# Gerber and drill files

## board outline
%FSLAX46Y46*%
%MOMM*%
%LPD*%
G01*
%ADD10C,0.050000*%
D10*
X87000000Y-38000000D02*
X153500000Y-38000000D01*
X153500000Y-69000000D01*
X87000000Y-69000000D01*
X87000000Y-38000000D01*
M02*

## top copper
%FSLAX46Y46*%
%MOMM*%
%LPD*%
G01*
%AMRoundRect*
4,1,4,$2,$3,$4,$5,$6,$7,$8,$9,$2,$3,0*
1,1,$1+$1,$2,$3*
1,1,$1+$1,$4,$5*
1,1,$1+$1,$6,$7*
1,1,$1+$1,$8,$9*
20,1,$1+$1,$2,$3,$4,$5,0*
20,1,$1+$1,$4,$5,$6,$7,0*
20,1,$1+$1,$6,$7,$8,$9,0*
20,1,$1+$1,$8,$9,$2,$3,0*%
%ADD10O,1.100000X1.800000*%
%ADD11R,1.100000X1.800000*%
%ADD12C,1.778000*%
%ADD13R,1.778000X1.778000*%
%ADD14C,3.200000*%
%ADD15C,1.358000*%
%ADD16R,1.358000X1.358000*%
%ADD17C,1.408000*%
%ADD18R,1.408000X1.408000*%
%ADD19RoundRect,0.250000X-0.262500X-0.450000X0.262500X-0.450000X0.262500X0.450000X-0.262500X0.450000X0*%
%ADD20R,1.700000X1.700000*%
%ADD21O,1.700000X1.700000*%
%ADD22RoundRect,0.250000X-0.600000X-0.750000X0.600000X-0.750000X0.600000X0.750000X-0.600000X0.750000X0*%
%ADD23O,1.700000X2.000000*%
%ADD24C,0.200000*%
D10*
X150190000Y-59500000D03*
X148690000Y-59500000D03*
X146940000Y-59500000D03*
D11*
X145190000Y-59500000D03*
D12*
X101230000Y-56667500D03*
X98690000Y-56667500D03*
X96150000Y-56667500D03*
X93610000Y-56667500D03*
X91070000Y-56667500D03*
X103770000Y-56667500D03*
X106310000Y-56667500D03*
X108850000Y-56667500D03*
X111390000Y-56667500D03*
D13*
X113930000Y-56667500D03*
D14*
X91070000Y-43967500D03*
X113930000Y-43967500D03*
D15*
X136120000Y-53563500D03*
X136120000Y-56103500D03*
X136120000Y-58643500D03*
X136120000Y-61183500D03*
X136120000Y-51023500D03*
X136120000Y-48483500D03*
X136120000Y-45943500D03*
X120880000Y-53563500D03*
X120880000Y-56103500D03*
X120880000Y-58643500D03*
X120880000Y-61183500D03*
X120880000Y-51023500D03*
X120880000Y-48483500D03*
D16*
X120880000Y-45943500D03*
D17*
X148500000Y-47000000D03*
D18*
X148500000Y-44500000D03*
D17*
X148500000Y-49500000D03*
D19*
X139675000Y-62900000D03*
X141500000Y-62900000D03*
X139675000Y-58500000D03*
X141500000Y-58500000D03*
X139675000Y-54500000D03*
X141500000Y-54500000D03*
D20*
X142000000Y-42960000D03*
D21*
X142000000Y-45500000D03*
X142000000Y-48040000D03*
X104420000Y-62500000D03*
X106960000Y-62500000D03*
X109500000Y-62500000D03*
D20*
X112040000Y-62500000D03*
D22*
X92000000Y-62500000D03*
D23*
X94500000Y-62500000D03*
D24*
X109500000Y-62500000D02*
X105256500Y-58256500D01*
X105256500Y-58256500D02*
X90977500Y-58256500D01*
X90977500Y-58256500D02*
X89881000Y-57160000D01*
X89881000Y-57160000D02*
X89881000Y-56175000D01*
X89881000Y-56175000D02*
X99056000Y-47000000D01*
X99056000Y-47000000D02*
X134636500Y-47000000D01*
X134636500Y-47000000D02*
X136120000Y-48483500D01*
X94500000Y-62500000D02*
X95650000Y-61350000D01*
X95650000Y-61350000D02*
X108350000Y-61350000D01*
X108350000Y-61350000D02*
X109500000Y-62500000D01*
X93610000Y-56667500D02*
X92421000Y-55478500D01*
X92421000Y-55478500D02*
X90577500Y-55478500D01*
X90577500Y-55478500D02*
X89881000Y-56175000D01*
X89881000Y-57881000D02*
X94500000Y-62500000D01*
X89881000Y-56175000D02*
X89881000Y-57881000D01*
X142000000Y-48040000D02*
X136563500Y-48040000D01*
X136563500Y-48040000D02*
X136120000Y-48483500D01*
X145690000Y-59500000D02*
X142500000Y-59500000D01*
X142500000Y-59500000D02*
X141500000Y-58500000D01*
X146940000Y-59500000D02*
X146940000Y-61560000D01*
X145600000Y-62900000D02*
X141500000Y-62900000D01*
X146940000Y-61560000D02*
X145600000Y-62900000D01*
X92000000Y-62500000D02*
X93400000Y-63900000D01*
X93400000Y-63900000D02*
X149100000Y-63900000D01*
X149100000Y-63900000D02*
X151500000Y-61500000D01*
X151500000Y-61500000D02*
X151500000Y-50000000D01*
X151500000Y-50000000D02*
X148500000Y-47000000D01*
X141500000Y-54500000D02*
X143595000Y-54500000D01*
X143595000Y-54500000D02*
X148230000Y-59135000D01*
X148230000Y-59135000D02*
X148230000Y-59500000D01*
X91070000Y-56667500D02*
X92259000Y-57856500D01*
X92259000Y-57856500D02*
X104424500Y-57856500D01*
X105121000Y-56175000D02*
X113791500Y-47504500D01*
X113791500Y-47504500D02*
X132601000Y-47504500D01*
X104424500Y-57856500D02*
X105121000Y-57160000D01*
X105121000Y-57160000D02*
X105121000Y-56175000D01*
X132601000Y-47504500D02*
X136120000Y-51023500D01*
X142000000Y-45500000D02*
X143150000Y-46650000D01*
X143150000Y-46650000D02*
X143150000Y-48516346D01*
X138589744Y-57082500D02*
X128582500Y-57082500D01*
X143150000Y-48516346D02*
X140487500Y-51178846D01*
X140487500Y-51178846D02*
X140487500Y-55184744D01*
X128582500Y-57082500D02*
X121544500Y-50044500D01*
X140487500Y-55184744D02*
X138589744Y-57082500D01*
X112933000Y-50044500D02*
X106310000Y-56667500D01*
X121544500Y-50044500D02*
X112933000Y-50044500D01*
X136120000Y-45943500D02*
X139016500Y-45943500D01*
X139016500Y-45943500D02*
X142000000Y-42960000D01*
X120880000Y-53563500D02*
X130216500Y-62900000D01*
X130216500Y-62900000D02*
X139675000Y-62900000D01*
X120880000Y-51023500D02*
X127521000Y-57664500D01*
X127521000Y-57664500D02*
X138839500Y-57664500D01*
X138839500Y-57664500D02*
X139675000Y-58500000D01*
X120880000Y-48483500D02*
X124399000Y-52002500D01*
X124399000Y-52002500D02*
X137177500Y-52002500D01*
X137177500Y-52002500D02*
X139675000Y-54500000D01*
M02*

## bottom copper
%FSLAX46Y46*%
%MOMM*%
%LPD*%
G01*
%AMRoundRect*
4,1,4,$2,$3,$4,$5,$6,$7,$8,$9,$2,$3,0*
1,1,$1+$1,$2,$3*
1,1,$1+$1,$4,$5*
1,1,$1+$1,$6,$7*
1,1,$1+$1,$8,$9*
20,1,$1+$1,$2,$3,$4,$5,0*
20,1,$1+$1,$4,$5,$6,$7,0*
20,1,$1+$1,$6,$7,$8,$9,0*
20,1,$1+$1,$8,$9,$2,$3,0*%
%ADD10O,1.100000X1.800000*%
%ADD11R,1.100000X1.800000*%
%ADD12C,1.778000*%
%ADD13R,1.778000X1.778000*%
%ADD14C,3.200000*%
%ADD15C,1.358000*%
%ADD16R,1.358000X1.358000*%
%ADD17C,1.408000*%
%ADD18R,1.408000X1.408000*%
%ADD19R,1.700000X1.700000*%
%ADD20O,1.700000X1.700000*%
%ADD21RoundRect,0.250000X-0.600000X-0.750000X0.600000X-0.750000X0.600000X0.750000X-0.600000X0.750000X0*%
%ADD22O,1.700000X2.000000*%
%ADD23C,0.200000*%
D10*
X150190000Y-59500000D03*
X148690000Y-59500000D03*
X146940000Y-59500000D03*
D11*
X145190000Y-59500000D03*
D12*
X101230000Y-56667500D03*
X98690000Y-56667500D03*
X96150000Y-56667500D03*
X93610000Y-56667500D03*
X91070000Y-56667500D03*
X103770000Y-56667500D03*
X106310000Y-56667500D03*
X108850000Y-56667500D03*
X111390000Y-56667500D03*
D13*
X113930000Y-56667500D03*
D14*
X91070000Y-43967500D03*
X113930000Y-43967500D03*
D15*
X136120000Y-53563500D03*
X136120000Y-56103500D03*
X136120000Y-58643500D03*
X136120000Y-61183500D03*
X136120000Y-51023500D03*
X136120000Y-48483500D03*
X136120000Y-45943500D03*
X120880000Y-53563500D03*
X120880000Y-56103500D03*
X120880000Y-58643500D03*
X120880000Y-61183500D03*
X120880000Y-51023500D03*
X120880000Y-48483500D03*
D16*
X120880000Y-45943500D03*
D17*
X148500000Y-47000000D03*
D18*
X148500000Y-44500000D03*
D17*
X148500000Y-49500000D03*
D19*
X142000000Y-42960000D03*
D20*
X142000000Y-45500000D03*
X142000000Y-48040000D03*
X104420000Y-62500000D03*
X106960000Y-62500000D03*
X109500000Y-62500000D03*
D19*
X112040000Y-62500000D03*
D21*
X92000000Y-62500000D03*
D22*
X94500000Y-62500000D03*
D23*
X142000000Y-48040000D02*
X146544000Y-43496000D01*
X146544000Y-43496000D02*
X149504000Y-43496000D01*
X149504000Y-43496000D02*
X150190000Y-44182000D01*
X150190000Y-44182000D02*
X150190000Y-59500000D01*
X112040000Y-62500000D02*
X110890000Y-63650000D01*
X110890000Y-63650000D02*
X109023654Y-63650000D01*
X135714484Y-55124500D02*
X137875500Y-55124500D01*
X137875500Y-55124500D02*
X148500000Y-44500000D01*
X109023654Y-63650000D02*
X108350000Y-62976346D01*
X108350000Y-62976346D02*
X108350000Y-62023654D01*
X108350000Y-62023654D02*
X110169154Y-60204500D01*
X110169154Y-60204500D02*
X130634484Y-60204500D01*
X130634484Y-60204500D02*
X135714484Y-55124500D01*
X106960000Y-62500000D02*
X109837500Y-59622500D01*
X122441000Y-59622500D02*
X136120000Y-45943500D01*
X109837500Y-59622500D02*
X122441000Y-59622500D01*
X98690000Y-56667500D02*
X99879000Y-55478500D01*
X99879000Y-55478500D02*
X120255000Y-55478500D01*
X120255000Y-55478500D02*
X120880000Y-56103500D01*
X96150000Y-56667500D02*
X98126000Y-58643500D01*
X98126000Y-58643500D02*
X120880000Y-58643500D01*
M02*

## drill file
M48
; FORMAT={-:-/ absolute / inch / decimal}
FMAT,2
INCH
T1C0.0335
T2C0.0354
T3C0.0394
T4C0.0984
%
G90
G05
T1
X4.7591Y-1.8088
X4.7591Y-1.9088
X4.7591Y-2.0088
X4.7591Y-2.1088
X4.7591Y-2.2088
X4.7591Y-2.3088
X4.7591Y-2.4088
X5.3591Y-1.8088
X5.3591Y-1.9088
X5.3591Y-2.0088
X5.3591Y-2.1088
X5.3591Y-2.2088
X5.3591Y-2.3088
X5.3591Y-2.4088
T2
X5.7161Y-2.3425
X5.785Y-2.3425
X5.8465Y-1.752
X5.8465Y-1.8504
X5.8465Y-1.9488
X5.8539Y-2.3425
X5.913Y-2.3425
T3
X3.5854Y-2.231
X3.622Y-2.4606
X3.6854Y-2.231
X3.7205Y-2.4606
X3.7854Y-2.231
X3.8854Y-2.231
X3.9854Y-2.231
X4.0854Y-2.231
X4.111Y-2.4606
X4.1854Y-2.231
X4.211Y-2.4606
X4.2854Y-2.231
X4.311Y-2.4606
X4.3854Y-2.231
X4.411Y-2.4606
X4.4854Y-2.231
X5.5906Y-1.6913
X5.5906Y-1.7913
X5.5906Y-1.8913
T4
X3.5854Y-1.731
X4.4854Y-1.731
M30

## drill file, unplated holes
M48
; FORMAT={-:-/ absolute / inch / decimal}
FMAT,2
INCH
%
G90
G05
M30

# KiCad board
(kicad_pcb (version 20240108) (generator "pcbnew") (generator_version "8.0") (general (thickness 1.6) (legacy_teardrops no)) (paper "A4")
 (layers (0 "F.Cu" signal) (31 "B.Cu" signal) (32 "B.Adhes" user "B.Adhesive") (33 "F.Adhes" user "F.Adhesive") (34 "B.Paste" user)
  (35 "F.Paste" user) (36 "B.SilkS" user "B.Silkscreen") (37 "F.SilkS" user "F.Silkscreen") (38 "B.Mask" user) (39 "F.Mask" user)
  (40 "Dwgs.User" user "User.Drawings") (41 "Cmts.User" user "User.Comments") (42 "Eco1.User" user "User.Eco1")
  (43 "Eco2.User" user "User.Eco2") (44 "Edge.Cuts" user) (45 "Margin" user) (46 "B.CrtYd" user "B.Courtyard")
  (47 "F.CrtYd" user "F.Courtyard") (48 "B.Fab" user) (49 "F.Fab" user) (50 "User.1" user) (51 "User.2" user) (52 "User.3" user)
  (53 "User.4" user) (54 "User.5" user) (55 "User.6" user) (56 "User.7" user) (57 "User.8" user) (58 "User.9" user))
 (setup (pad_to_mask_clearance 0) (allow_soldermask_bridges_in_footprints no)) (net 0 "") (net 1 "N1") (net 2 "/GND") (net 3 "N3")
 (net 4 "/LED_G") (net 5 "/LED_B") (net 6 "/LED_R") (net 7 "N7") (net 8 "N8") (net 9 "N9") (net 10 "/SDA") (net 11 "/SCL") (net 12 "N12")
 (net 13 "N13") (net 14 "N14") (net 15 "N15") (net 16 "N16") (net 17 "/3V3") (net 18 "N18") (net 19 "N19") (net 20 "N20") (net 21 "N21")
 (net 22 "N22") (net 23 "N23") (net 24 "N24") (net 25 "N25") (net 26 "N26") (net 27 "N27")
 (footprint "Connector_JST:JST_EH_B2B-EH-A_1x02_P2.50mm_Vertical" (layer "F.Cu") (at 92 62.5)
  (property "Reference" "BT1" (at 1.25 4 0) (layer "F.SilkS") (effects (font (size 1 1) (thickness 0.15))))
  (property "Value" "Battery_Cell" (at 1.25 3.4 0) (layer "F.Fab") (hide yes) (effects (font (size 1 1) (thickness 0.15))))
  (pad "1" thru_hole roundrect (at 0 0) (size 1.7 2) (drill 1) (layers "*.Cu" "*.Mask") (remove_unused_layers no)
   (roundrect_rratio 0.147059) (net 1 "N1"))
  (pad "2" thru_hole oval (at 2.5 0) (size 1.7 2) (drill 1) (layers "*.Cu" "*.Mask") (remove_unused_layers no) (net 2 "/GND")))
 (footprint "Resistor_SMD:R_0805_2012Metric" (layer "F.Cu") (at 140.5875 58.5)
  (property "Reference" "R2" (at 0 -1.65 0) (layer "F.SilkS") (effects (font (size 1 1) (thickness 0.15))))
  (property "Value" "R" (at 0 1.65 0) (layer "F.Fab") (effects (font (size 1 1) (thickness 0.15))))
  (pad "1" smd roundrect (at -0.9125 0) (size 1.025 1.4) (layers "F.Cu" "F.Paste" "F.Mask") (roundrect_rratio 0.243902) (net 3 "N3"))
  (pad "2" smd roundrect (at 0.9125 0) (size 1.025 1.4) (layers "F.Cu" "F.Paste" "F.Mask") (roundrect_rratio 0.243902) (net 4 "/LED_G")))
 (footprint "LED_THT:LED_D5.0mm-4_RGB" (layer "F.Cu") (at 145.69 59.5)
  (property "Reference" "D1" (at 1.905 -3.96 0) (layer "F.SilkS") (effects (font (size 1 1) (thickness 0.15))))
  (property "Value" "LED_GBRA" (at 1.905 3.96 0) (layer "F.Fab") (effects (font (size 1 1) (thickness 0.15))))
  (pad "1" thru_hole rect (at -0.5 0) (size 1.1 1.8) (drill 0.9) (layers "*.Cu" "*.Mask") (remove_unused_layers no) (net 4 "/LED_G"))
  (pad "2" thru_hole oval (at 1.25 0) (size 1.1 1.8) (drill 0.9) (layers "*.Cu" "*.Mask") (remove_unused_layers no) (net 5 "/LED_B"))
  (pad "3" thru_hole oval (at 3 0) (size 1.1 1.8) (drill 0.9) (layers "*.Cu" "*.Mask") (remove_unused_layers no) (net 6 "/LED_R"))
  (pad "4" thru_hole oval (at 4.5 0) (size 1.1 1.8) (drill 0.9) (layers "*.Cu" "*.Mask") (remove_unused_layers no) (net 2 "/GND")))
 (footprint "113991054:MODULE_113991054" (layer "F.Cu") (at 128.5 53.5)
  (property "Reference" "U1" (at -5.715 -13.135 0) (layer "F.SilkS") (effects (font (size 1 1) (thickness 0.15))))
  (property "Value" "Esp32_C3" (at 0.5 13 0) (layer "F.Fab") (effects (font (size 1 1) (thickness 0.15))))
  (pad "1" thru_hole rect (at -7.62 -7.5565) (size 1.358 1.358) (drill 0.85) (layers "*.Cu" "*.Mask") (remove_unused_layers no) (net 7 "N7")
   (solder_mask_margin 0.102))
  (pad "2" thru_hole circle (at -7.62 -5.0165) (size 1.358 1.358) (drill 0.85) (layers "*.Cu" "*.Mask") (remove_unused_layers no)
   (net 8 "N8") (solder_mask_margin 0.102))
  (pad "3" thru_hole circle (at -7.62 -2.4765) (size 1.358 1.358) (drill 0.85) (layers "*.Cu" "*.Mask") (remove_unused_layers no)
   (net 3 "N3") (solder_mask_margin 0.102))
  (pad "4" thru_hole circle (at -7.62 0.0635) (size 1.358 1.358) (drill 0.85) (layers "*.Cu" "*.Mask") (remove_unused_layers no)
   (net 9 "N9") (solder_mask_margin 0.102))
  (pad "5" thru_hole circle (at -7.62 2.6035) (size 1.358 1.358) (drill 0.85) (layers "*.Cu" "*.Mask") (remove_unused_layers no)
   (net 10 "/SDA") (solder_mask_margin 0.102))
  (pad "6" thru_hole circle (at -7.62 5.1435) (size 1.358 1.358) (drill 0.85) (layers "*.Cu" "*.Mask") (remove_unused_layers no)
   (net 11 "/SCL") (solder_mask_margin 0.102))
  (pad "7" thru_hole circle (at -7.62 7.6835) (size 1.358 1.358) (drill 0.85) (layers "*.Cu" "*.Mask") (remove_unused_layers no)
   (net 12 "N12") (solder_mask_margin 0.102))
  (pad "8" thru_hole circle (at 7.62 7.6835) (size 1.358 1.358) (drill 0.85) (layers "*.Cu" "*.Mask") (remove_unused_layers no)
   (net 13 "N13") (solder_mask_margin 0.102))
  (pad "9" thru_hole circle (at 7.62 5.1435) (size 1.358 1.358) (drill 0.85) (layers "*.Cu" "*.Mask") (remove_unused_layers no)
   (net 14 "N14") (solder_mask_margin 0.102))
  (pad "10" thru_hole circle (at 7.62 2.6035) (size 1.358 1.358) (drill 0.85) (layers "*.Cu" "*.Mask") (remove_unused_layers no)
   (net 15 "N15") (solder_mask_margin 0.102))
  (pad "11" thru_hole circle (at 7.62 0.0635) (size 1.358 1.358) (drill 0.85) (layers "*.Cu" "*.Mask") (remove_unused_layers no)
   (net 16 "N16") (solder_mask_margin 0.102))
  (pad "12" thru_hole circle (at 7.62 -2.4765) (size 1.358 1.358) (drill 0.85) (layers "*.Cu" "*.Mask") (remove_unused_layers no)
   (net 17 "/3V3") (solder_mask_margin 0.102))
  (pad "13" thru_hole circle (at 7.62 -5.0165) (size 1.358 1.358) (drill 0.85) (layers "*.Cu" "*.Mask") (remove_unused_layers no)
   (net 2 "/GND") (solder_mask_margin 0.102))
  (pad "14" thru_hole circle (at 7.62 -7.5565) (size 1.358 1.358) (drill 0.85) (layers "*.Cu" "*.Mask") (remove_unused_layers no)
   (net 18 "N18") (solder_mask_margin 0.102)))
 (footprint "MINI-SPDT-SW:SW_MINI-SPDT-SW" (layer "F.Cu") (at 148.5 47 -90)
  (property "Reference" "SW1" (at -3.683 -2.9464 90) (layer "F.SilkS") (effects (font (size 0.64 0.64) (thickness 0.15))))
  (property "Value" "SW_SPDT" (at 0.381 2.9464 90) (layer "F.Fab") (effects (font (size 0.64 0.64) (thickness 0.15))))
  (pad "1" thru_hole rect (at -2.5 0 270) (size 1.408 1.408) (drill 0.9) (layers "*.Cu" "*.Mask") (remove_unused_layers no) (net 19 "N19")
   (solder_mask_margin 0.102))
  (pad "2" thru_hole circle (at 0 0 270) (size 1.408 1.408) (drill 0.9) (layers "*.Cu" "*.Mask") (remove_unused_layers no) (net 1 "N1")
   (solder_mask_margin 0.102))
  (pad "3" thru_hole circle (at 2.5 0 270) (size 1.408 1.408) (drill 0.9) (layers "*.Cu" "*.Mask") (remove_unused_layers no) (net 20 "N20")
   (solder_mask_margin 0.102)))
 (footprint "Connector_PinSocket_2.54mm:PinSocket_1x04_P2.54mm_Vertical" (layer "F.Cu") (at 112.04 62.5 -90)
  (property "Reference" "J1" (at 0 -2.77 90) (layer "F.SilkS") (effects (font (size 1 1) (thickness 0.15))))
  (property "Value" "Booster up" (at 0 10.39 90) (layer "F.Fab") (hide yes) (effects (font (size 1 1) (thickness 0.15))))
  (pad "1" thru_hole rect (at 0 0 270) (size 1.7 1.7) (drill 1) (layers "*.Cu" "*.Mask") (remove_unused_layers no) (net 19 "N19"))
  (pad "2" thru_hole oval (at 0 2.54 270) (size 1.7 1.7) (drill 1) (layers "*.Cu" "*.Mask") (remove_unused_layers no) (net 2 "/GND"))
  (pad "3" thru_hole oval (at 0 5.08 270) (size 1.7 1.7) (drill 1) (layers "*.Cu" "*.Mask") (remove_unused_layers no) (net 18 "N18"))
  (pad "4" thru_hole oval (at 0 7.62 270) (size 1.7 1.7) (drill 1) (layers "*.Cu" "*.Mask") (remove_unused_layers no) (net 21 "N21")))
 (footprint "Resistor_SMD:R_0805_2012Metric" (layer "F.Cu") (at 140.5875 54.5)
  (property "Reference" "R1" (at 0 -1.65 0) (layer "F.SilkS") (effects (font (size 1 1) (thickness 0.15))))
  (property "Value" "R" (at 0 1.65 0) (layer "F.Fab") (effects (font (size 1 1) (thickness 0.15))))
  (pad "1" smd roundrect (at -0.9125 0) (size 1.025 1.4) (layers "F.Cu" "F.Paste" "F.Mask") (roundrect_rratio 0.243902) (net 8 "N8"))
  (pad "2" smd roundrect (at 0.9125 0) (size 1.025 1.4) (layers "F.Cu" "F.Paste" "F.Mask") (roundrect_rratio 0.243902) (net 6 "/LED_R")))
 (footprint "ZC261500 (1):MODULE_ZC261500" (layer "F.Cu") (at 102.5 50)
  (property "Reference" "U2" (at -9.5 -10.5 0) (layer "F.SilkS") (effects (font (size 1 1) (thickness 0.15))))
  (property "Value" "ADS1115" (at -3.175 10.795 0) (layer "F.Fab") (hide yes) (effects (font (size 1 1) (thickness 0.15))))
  (pad "1" thru_hole rect (at 11.43 6.6675) (size 1.778 1.778) (drill 1) (layers "*.Cu" "*.Mask") (remove_unused_layers no) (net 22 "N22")
   (solder_mask_margin 0.102))
  (pad "2" thru_hole circle (at 8.89 6.6675) (size 1.778 1.778) (drill 1) (layers "*.Cu" "*.Mask") (remove_unused_layers no) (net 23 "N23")
   (solder_mask_margin 0.102))
  (pad "3" thru_hole circle (at 6.35 6.6675) (size 1.778 1.778) (drill 1) (layers "*.Cu" "*.Mask") (remove_unused_layers no) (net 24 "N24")
   (solder_mask_margin 0.102))
  (pad "4" thru_hole circle (at 3.81 6.6675) (size 1.778 1.778) (drill 1) (layers "*.Cu" "*.Mask") (remove_unused_layers no) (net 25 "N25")
   (solder_mask_margin 0.102))
  (pad "5" thru_hole circle (at 1.27 6.6675) (size 1.778 1.778) (drill 1) (layers "*.Cu" "*.Mask") (remove_unused_layers no) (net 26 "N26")
   (solder_mask_margin 0.102))
  (pad "6" thru_hole circle (at -1.27 6.6675) (size 1.778 1.778) (drill 1) (layers "*.Cu" "*.Mask") (remove_unused_layers no) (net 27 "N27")
   (solder_mask_margin 0.102))
  (pad "7" thru_hole circle (at -3.81 6.6675) (size 1.778 1.778) (drill 1) (layers "*.Cu" "*.Mask") (remove_unused_layers no)
   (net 10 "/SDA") (solder_mask_margin 0.102))
  (pad "8" thru_hole circle (at -6.35 6.6675) (size 1.778 1.778) (drill 1) (layers "*.Cu" "*.Mask") (remove_unused_layers no)
   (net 11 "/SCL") (solder_mask_margin 0.102))
  (pad "9" thru_hole circle (at -8.89 6.6675) (size 1.778 1.778) (drill 1) (layers "*.Cu" "*.Mask") (remove_unused_layers no) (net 2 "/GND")
   (solder_mask_margin 0.102))
  (pad "10" thru_hole circle (at -11.43 6.6675) (size 1.778 1.778) (drill 1) (layers "*.Cu" "*.Mask") (remove_unused_layers no)
   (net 17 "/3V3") (solder_mask_margin 0.102))
  (pad "P1" thru_hole circle (at -11.43 -6.0325) (size 3.2 3.2) (drill 2.5) (layers "*.Cu" "*.Mask") (remove_unused_layers no)
   (solder_mask_margin 0.102))
  (pad "P2" thru_hole circle (at 11.43 -6.0325) (size 3.2 3.2) (drill 2.5) (layers "*.Cu" "*.Mask") (remove_unused_layers no)
   (solder_mask_margin 0.102)))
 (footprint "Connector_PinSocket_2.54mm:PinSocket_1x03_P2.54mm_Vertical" (layer "F.Cu") (at 142 42.96)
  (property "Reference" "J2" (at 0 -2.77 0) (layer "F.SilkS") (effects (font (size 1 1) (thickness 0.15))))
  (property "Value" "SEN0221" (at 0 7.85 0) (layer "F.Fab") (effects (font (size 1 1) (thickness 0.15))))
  (pad "1" thru_hole rect (at 0 0) (size 1.7 1.7) (drill 1) (layers "*.Cu" "*.Mask") (remove_unused_layers no) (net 18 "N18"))
  (pad "2" thru_hole oval (at 0 2.54) (size 1.7 1.7) (drill 1) (layers "*.Cu" "*.Mask") (remove_unused_layers no) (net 25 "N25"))
  (pad "3" thru_hole oval (at 0 5.08) (size 1.7 1.7) (drill 1) (layers "*.Cu" "*.Mask") (remove_unused_layers no) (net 2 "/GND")))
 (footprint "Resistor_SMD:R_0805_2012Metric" (layer "F.Cu") (at 140.5875 62.9)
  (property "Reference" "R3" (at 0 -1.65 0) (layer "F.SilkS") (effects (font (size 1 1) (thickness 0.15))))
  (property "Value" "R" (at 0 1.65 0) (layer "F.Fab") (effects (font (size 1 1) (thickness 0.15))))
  (pad "1" smd roundrect (at -0.9125 0) (size 1.025 1.4) (layers "F.Cu" "F.Paste" "F.Mask") (roundrect_rratio 0.243902) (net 9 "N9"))
  (pad "2" smd roundrect (at 0.9125 0) (size 1.025 1.4) (layers "F.Cu" "F.Paste" "F.Mask") (roundrect_rratio 0.243902) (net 5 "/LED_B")))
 (gr_rect (start 87 38) (end 153.5 69) (stroke (width 0.05) (type default)) (fill none) (layer "Edge.Cuts"))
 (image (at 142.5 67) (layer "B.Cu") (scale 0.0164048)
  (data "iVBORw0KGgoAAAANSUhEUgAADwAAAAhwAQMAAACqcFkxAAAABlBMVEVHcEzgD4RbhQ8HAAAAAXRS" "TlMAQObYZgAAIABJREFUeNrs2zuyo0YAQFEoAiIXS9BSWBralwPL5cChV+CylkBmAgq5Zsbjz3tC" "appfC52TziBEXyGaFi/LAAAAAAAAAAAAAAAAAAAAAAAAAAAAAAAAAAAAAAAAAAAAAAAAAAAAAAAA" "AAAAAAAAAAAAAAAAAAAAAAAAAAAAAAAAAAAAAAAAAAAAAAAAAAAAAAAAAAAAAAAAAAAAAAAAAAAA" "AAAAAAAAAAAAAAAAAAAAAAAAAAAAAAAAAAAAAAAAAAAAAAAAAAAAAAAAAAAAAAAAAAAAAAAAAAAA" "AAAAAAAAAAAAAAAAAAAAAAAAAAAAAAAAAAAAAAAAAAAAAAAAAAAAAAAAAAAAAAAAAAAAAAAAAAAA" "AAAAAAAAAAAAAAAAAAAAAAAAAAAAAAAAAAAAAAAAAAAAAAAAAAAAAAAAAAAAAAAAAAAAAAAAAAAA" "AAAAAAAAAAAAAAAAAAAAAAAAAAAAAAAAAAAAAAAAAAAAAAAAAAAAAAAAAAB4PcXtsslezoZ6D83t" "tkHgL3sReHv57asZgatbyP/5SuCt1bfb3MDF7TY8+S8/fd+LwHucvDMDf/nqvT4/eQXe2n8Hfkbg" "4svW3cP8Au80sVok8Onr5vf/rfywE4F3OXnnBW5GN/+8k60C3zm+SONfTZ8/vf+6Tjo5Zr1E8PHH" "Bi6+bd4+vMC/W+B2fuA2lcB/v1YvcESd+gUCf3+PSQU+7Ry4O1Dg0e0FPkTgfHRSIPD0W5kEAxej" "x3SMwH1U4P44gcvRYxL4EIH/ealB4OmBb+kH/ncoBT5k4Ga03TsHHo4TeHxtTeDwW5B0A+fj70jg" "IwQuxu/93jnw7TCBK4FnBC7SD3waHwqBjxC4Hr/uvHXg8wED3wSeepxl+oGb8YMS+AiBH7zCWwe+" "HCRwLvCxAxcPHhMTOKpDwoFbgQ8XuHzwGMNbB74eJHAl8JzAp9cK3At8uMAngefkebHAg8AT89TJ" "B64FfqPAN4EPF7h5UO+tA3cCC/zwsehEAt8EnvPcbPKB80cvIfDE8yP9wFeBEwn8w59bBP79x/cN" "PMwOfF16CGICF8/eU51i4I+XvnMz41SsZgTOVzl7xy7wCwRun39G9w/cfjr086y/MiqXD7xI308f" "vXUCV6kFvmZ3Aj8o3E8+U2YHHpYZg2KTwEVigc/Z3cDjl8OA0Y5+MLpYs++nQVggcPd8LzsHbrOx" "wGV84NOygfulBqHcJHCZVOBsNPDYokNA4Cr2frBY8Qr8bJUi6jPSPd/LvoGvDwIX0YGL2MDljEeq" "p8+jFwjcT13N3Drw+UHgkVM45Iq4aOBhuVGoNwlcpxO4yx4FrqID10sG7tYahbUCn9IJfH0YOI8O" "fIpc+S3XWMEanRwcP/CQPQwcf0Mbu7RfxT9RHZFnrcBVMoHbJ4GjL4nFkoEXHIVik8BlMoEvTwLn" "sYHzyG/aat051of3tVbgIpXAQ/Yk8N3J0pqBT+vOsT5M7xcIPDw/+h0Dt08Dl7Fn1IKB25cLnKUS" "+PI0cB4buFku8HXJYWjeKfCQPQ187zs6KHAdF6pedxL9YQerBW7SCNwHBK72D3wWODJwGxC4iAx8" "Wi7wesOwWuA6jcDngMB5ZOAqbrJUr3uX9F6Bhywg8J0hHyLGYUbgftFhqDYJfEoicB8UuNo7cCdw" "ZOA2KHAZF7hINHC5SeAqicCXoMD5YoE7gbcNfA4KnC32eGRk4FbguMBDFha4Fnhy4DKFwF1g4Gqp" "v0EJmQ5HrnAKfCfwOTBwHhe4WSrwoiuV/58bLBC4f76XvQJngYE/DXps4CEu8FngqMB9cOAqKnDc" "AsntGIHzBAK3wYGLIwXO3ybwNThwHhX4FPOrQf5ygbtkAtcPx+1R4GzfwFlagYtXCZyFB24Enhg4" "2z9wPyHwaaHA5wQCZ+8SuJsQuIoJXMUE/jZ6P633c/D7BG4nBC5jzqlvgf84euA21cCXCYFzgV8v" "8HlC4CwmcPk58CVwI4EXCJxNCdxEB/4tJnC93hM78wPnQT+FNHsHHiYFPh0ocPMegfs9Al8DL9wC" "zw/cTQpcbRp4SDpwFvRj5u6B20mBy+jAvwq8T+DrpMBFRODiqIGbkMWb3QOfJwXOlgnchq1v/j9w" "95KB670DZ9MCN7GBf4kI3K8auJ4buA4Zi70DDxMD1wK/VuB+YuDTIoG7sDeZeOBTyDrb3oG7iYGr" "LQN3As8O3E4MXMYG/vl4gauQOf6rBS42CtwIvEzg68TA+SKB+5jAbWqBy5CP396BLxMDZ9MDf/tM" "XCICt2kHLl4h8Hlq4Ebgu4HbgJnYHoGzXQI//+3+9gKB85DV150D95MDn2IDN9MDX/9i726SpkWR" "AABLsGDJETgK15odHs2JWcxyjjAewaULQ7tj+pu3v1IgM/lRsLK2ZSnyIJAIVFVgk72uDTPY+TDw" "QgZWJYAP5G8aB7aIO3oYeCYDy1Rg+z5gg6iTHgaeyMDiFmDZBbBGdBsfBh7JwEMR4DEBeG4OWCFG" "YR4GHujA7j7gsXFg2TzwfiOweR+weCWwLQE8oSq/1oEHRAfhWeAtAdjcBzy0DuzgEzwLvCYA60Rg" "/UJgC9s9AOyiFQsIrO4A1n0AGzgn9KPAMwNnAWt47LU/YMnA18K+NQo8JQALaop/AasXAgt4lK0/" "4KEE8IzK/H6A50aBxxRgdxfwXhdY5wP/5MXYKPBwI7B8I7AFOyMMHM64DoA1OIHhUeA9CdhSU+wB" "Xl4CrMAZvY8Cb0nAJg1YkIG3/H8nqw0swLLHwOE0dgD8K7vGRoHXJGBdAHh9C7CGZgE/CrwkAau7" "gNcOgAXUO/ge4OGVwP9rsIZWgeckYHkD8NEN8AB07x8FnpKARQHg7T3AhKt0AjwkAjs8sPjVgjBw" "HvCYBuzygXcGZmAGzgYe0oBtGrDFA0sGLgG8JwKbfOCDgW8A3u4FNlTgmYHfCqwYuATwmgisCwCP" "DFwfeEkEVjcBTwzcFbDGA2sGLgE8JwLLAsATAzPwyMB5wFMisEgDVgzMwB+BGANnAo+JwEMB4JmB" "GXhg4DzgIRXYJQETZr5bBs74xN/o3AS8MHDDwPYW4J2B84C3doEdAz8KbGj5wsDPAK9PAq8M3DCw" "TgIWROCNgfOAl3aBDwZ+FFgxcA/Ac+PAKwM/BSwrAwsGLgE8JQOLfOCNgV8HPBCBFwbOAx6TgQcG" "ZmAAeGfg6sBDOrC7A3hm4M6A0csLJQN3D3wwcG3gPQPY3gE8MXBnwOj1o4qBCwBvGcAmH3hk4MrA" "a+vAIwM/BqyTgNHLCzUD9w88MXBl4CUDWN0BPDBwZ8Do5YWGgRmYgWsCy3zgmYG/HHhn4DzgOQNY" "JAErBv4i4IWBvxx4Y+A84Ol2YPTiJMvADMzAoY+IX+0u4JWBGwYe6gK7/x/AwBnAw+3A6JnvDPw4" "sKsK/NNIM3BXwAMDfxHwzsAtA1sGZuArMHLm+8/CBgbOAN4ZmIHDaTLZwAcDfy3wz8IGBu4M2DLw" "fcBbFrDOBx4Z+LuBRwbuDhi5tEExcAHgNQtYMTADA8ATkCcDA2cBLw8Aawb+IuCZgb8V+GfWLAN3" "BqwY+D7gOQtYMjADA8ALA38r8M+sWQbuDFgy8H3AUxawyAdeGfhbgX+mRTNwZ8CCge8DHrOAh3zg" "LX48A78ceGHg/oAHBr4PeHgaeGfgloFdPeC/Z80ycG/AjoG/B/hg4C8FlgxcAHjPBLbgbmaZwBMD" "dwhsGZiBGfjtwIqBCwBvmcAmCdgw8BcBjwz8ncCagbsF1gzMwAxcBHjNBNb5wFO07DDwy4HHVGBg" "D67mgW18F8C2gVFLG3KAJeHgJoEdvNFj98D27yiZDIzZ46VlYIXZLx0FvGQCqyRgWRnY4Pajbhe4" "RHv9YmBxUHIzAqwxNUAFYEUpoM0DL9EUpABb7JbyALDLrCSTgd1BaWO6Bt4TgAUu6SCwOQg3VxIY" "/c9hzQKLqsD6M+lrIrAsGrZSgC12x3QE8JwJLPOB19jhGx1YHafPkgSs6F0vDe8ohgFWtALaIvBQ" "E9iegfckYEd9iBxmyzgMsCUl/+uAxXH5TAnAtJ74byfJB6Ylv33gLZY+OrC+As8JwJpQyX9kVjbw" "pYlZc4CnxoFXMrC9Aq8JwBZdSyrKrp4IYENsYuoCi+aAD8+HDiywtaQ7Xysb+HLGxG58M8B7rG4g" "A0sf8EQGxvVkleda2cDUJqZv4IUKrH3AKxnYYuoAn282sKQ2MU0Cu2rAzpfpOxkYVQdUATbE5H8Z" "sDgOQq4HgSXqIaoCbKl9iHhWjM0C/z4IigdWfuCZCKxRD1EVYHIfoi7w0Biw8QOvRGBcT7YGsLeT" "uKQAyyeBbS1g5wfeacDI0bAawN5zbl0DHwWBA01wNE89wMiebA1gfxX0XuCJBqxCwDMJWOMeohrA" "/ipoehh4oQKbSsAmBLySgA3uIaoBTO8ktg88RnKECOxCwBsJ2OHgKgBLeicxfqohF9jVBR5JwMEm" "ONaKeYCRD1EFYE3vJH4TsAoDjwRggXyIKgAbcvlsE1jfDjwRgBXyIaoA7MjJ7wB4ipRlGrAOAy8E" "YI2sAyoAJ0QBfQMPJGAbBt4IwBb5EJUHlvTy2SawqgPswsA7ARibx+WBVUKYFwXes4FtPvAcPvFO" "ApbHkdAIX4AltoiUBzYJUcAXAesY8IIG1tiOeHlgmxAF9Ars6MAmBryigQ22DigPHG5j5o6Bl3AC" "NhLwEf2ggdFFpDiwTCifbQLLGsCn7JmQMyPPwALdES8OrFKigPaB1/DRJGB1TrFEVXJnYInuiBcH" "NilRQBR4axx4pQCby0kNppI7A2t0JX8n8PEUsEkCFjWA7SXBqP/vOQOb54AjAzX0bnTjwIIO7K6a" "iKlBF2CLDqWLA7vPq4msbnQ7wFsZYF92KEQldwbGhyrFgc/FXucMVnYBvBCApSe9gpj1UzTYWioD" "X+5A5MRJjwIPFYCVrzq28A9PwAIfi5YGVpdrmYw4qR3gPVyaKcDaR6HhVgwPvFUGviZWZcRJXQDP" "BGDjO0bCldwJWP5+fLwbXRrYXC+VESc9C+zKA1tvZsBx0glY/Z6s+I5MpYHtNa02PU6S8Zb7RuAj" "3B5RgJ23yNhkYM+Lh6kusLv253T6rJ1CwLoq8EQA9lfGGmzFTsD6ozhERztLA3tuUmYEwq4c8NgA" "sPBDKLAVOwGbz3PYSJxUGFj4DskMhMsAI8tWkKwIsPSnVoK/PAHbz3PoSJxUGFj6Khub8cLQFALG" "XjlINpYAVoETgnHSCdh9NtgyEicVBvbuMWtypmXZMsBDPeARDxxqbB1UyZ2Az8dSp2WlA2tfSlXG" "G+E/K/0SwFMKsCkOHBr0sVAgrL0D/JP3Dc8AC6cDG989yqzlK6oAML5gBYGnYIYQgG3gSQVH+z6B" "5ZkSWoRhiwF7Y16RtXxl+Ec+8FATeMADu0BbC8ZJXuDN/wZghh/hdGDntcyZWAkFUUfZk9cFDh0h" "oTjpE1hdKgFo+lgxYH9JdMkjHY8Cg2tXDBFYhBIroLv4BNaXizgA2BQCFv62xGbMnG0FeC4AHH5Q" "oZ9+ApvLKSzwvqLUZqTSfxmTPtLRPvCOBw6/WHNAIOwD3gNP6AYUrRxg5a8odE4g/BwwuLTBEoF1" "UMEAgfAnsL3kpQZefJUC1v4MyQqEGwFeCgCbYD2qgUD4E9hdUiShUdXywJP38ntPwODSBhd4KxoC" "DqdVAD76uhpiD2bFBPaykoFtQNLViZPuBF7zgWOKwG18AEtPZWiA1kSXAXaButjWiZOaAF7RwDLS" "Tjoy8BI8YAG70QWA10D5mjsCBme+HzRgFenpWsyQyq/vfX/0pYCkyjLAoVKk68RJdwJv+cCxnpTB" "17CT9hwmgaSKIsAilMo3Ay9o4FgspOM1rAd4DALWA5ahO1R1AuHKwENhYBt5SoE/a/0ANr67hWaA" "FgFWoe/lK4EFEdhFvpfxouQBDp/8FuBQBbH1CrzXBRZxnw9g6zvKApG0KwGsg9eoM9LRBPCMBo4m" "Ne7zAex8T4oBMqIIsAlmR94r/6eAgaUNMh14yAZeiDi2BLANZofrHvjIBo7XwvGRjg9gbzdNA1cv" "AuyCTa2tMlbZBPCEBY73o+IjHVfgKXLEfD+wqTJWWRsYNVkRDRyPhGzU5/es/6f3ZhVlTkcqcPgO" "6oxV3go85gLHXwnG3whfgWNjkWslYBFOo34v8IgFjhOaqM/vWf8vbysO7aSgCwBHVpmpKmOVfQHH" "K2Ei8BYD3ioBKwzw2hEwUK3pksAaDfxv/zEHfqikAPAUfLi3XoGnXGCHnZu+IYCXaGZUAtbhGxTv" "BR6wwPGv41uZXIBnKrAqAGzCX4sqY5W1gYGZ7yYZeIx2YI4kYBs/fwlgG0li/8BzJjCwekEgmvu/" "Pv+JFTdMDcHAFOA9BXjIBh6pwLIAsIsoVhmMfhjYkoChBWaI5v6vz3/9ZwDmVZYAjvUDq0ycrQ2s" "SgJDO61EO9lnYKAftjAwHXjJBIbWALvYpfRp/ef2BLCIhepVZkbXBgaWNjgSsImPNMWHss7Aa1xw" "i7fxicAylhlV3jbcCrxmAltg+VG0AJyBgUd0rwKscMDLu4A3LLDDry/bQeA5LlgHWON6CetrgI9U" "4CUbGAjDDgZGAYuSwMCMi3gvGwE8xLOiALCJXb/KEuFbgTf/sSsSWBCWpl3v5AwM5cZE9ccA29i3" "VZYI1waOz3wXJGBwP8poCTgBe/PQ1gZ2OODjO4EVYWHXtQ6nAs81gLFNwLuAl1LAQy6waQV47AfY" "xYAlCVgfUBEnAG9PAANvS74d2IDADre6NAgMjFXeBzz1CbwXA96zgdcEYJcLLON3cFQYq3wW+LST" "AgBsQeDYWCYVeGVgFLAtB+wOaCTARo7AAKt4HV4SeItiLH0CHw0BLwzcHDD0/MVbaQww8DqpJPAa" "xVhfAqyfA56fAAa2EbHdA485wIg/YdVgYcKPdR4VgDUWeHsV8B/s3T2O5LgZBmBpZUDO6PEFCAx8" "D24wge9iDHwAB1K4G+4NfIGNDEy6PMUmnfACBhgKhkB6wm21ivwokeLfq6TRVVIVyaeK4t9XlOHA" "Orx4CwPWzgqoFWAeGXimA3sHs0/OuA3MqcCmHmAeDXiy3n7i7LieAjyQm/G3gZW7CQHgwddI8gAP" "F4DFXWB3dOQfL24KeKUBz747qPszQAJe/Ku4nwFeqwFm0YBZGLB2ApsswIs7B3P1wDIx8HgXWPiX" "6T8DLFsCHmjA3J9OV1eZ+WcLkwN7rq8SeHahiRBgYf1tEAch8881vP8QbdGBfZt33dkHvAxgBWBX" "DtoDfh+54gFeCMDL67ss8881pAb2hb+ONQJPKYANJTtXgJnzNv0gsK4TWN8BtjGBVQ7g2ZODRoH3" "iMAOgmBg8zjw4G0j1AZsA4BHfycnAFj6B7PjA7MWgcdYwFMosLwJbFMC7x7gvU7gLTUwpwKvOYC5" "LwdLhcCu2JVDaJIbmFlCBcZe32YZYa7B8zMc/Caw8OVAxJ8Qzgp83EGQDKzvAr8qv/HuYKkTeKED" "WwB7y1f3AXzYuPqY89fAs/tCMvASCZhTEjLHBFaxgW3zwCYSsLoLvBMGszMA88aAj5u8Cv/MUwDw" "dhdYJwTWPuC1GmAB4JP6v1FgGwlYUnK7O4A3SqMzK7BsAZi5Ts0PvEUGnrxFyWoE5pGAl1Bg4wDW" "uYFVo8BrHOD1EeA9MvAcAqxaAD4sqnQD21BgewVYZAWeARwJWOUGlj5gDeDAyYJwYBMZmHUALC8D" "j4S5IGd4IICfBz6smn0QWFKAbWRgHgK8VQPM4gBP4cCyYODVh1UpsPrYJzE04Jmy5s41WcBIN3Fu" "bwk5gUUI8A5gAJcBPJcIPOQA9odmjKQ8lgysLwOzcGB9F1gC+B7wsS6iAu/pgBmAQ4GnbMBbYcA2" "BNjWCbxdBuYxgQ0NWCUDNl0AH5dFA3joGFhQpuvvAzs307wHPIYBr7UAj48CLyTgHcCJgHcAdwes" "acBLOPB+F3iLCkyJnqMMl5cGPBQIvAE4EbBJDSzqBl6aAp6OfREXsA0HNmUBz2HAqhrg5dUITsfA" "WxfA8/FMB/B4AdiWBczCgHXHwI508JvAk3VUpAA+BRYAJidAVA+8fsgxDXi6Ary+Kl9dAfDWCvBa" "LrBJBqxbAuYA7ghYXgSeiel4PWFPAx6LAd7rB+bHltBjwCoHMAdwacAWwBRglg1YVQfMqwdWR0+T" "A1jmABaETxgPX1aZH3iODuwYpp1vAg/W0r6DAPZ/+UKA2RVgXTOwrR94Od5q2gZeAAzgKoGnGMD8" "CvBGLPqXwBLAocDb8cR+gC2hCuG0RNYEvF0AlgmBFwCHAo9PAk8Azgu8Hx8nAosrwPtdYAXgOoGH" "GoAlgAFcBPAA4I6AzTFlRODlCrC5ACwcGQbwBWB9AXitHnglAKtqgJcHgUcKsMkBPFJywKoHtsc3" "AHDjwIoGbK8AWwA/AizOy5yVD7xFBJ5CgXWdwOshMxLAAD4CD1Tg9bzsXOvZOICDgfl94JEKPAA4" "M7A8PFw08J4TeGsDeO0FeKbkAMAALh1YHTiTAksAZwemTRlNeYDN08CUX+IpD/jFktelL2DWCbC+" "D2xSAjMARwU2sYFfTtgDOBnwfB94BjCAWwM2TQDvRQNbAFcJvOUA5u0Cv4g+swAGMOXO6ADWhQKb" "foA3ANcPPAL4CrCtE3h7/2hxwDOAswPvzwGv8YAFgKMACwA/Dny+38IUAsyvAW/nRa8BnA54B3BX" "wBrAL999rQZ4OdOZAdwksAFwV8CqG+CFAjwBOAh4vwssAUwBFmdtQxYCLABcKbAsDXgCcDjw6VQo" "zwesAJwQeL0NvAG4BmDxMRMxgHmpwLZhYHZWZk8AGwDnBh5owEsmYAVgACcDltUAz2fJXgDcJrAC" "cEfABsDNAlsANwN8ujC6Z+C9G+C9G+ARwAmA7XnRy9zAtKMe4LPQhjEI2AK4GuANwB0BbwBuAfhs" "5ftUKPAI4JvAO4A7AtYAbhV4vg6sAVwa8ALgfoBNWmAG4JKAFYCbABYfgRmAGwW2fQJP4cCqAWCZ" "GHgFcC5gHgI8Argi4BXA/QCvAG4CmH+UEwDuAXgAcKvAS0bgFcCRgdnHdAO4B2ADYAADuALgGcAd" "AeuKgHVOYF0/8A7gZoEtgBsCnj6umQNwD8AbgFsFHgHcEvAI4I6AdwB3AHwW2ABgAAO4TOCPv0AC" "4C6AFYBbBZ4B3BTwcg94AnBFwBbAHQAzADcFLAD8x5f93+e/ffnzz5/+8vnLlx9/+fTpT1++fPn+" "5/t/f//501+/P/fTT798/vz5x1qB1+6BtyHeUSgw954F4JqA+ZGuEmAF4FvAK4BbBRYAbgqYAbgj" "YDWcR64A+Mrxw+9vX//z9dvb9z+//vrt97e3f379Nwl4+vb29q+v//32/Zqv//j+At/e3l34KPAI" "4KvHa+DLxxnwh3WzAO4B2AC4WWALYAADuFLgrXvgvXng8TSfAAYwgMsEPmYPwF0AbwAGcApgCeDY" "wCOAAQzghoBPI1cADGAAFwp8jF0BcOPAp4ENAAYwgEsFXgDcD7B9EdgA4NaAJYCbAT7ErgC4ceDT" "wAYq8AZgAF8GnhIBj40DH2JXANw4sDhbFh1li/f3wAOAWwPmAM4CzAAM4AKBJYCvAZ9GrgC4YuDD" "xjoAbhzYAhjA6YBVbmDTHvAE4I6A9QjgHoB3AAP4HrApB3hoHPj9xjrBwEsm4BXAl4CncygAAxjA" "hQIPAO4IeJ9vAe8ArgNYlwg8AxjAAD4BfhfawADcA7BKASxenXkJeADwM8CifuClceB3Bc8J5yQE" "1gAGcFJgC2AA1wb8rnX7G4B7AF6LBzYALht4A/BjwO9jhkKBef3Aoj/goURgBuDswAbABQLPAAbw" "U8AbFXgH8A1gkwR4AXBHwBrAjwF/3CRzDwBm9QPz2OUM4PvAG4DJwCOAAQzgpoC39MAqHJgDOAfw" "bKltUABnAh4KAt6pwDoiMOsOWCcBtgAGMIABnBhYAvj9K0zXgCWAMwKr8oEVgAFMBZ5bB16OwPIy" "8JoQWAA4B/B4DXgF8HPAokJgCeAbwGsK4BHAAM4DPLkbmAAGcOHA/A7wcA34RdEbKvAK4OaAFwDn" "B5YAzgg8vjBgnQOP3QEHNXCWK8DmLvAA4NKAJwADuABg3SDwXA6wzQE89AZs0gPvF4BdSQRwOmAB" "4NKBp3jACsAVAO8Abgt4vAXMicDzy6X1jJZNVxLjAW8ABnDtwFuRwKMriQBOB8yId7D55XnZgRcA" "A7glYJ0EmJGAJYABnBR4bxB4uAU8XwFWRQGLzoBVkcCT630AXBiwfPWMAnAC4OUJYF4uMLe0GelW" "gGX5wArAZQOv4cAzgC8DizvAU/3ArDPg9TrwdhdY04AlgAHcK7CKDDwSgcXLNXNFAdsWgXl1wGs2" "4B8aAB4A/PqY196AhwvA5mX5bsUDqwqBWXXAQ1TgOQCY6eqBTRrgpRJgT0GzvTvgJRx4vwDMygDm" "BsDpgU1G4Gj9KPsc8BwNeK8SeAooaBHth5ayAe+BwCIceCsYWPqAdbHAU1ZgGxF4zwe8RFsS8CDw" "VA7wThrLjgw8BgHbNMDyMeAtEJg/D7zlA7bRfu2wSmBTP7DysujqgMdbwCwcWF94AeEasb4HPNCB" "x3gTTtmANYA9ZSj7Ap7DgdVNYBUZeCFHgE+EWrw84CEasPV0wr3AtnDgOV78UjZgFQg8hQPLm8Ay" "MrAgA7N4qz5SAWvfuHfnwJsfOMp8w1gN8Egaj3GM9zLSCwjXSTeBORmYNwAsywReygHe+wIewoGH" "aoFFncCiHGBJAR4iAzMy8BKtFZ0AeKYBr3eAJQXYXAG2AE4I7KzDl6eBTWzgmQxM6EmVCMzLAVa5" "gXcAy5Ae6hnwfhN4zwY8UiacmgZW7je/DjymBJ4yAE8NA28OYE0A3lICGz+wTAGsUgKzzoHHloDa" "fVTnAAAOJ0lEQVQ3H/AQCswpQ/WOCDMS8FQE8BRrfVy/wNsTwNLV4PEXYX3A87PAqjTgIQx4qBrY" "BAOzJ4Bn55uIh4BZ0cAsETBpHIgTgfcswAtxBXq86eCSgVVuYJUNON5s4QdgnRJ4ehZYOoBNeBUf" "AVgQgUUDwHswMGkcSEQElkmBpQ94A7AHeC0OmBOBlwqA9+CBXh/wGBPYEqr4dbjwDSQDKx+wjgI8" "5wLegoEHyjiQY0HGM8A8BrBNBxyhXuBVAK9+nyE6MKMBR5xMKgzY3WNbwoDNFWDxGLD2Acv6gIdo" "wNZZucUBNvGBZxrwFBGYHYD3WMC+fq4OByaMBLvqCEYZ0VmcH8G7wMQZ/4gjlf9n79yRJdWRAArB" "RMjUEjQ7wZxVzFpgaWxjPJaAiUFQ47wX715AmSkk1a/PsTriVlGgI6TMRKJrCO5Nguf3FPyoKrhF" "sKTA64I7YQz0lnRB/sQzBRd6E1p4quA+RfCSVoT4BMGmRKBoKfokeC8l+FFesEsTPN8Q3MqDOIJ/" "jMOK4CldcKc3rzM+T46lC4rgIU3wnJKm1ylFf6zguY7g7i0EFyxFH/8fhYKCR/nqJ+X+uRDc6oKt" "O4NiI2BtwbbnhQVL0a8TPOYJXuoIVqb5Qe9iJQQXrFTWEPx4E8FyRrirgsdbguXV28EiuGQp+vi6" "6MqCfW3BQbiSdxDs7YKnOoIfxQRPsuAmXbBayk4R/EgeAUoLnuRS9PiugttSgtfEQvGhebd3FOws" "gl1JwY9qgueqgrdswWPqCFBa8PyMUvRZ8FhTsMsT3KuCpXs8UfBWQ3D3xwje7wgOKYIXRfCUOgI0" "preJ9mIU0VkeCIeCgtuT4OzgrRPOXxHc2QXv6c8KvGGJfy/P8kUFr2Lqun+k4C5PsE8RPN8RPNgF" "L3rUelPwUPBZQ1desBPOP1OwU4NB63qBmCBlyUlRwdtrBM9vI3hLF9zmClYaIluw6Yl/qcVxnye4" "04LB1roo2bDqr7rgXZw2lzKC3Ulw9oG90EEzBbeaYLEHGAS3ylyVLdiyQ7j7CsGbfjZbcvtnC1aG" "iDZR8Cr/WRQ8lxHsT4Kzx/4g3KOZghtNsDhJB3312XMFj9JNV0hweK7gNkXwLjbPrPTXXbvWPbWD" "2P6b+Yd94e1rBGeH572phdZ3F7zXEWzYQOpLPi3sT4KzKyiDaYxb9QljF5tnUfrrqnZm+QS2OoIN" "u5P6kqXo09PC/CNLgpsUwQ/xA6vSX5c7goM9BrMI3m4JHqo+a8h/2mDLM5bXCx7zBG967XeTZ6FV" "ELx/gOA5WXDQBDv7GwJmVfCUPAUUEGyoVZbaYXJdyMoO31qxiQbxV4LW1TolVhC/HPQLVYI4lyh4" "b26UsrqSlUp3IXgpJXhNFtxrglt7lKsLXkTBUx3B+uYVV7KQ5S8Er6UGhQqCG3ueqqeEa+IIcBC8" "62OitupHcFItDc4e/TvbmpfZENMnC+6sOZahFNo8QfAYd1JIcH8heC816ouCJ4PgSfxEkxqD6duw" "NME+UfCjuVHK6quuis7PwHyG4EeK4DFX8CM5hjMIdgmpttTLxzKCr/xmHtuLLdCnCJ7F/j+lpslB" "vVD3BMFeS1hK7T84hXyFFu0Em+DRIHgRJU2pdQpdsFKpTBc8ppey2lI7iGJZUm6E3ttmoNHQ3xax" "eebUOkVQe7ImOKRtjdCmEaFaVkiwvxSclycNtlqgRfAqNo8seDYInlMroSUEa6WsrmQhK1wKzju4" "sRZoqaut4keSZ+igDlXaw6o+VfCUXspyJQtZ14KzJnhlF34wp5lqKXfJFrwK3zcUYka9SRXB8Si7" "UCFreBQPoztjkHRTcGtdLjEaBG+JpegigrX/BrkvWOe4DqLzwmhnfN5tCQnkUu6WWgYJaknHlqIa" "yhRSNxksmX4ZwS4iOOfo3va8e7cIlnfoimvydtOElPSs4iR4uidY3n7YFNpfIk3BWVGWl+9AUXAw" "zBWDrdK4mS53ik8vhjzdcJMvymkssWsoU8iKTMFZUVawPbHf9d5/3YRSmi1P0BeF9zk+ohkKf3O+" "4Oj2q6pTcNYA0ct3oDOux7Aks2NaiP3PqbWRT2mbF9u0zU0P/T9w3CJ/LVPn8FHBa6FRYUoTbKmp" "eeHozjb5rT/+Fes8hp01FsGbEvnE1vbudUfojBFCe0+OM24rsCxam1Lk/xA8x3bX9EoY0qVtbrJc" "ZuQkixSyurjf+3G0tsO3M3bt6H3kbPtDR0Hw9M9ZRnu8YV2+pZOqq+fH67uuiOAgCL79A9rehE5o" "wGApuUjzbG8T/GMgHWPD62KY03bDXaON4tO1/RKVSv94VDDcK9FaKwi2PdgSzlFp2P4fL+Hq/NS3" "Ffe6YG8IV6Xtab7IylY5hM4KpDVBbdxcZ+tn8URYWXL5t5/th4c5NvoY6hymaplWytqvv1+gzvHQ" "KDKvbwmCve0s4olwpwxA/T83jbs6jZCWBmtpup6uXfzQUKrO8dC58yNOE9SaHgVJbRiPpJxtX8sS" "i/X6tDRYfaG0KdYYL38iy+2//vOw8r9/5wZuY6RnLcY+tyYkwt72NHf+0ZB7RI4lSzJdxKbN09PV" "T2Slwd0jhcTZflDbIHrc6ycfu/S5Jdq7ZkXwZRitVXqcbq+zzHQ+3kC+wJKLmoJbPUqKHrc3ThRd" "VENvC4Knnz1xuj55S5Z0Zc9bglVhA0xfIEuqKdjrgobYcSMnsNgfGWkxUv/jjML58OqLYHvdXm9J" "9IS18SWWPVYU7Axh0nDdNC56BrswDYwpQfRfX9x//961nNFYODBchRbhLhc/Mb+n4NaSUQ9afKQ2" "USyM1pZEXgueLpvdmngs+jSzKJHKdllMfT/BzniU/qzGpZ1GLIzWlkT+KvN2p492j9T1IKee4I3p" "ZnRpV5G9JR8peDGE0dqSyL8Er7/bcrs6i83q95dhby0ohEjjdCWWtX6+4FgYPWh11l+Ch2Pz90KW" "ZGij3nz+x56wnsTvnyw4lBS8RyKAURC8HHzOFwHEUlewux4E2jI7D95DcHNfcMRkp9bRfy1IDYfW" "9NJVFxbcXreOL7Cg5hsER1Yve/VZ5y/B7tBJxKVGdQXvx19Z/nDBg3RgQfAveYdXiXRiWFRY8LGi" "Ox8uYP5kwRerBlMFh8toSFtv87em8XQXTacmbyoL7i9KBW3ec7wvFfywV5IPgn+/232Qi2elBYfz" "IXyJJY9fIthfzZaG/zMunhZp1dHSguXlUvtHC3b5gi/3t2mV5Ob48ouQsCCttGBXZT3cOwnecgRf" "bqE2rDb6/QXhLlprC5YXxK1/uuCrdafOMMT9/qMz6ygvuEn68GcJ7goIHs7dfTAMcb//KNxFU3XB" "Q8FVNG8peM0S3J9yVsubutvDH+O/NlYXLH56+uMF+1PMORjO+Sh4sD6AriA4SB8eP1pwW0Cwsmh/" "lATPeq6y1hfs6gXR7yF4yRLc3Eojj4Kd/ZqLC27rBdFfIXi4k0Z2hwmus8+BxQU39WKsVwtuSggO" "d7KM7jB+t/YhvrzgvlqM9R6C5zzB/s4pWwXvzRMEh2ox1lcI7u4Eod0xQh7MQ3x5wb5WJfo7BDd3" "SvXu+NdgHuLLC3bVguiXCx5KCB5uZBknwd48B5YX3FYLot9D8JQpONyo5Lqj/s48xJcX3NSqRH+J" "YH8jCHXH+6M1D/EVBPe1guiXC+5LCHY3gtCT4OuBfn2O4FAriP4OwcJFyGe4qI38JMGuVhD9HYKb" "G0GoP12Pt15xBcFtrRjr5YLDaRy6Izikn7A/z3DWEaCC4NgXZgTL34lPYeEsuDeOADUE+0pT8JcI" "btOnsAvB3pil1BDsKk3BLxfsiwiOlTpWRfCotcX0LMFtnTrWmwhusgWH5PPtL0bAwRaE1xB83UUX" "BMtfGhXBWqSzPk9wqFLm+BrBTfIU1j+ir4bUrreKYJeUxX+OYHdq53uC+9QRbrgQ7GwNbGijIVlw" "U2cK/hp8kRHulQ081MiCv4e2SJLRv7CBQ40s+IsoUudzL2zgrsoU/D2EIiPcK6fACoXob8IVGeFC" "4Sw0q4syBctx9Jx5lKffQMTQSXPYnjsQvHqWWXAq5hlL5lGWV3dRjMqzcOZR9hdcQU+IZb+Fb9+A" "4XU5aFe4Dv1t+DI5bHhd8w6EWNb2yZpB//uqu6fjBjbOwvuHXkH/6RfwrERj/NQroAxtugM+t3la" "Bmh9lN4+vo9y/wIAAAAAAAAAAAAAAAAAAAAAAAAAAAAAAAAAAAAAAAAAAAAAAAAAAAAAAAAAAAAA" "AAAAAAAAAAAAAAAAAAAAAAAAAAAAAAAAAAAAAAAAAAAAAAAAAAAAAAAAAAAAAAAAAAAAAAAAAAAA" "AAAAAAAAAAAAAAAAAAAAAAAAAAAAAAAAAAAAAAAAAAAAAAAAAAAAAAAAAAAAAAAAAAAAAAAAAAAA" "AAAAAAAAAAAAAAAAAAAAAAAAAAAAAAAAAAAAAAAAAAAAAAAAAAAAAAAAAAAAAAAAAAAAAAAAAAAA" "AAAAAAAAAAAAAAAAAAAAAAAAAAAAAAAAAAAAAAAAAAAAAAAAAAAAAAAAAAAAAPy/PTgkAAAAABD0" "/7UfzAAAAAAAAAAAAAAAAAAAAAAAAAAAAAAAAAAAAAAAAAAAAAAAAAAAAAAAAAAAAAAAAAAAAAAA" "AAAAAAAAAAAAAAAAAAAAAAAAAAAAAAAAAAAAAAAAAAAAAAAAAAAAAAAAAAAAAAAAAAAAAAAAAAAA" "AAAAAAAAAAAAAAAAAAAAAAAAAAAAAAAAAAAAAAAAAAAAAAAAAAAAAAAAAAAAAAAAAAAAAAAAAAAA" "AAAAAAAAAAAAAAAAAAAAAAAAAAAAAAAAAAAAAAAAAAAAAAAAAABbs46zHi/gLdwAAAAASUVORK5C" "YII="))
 (segment (start 89.881 56.175) (end 89.881 57.881) (width 0.2) (layer "F.Cu") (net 2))
 (segment (start 89.881 56.175) (end 99.056 47) (width 0.2) (layer "F.Cu") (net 2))
 (segment (start 89.881 57.881) (end 94.5 62.5) (width 0.2) (layer "F.Cu") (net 2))
 (segment (start 94.5 62.5) (end 95.65 61.35) (width 0.2) (layer "F.Cu") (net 2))
 (segment (start 90.9775 58.2565) (end 89.881 57.16) (width 0.2) (layer "F.Cu") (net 2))
 (segment (start 99.056 47) (end 134.6365 47) (width 0.2) (layer "F.Cu") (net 2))
 (segment (start 92.421 55.4785) (end 90.5775 55.4785) (width 0.2) (layer "F.Cu") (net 2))
 (segment (start 95.65 61.35) (end 108.35 61.35) (width 0.2) (layer "F.Cu") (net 2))
 (segment (start 109.5 62.5) (end 105.2565 58.2565) (width 0.2) (layer "F.Cu") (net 2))
 (segment (start 142 48.04) (end 136.5635 48.04) (width 0.2) (layer "F.Cu") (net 2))
 (segment (start 89.881 57.16) (end 89.881 56.175) (width 0.2) (layer "F.Cu") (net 2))
 (segment (start 105.2565 58.2565) (end 90.9775 58.2565) (width 0.2) (layer "F.Cu") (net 2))
 (segment (start 136.5635 48.04) (end 136.12 48.4835) (width 0.2) (layer "F.Cu") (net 2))
 (segment (start 108.35 61.35) (end 109.5 62.5) (width 0.2) (layer "F.Cu") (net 2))
 (segment (start 90.5775 55.4785) (end 89.881 56.175) (width 0.2) (layer "F.Cu") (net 2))
 (segment (start 93.61 56.6675) (end 92.421 55.4785) (width 0.2) (layer "F.Cu") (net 2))
 (segment (start 134.6365 47) (end 136.12 48.4835) (width 0.2) (layer "F.Cu") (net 2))
 (segment (start 150.19 44.182) (end 150.19 59.5) (width 0.2) (layer "B.Cu") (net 2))
 (segment (start 142 48.04) (end 146.544 43.496) (width 0.2) (layer "B.Cu") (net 2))
 (segment (start 149.504 43.496) (end 150.19 44.182) (width 0.2) (layer "B.Cu") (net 2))
 (segment (start 146.544 43.496) (end 149.504 43.496) (width 0.2) (layer "B.Cu") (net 2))
 (segment (start 92 62.5) (end 93.4 63.9) (width 0.2) (layer "F.Cu") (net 1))
 (segment (start 151.5 61.5) (end 151.5 50) (width 0.2) (layer "F.Cu") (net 1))
 (segment (start 93.4 63.9) (end 149.1 63.9) (width 0.2) (layer "F.Cu") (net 1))
 (segment (start 149.1 63.9) (end 151.5 61.5) (width 0.2) (layer "F.Cu") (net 1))
 (segment (start 151.5 50) (end 148.5 47) (width 0.2) (layer "F.Cu") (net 1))
 (segment (start 142.5 59.5) (end 141.5 58.5) (width 0.2) (layer "F.Cu") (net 4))
 (segment (start 145.69 59.5) (end 142.5 59.5) (width 0.2) (layer "F.Cu") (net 4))
 (segment (start 148.23 59.135) (end 148.23 59.5) (width 0.2) (layer "F.Cu") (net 6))
 (segment (start 141.5 54.5) (end 143.595 54.5) (width 0.2) (layer "F.Cu") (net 6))
 (segment (start 143.595 54.5) (end 148.23 59.135) (width 0.2) (layer "F.Cu") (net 6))
 (segment (start 146.94 61.56) (end 145.6 62.9) (width 0.2) (layer "F.Cu") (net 5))
 (segment (start 145.6 62.9) (end 141.5 62.9) (width 0.2) (layer "F.Cu") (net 5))
 (segment (start 146.94 59.5) (end 146.94 61.56) (width 0.2) (layer "F.Cu") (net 5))
 (segment (start 135.714484 55.1245) (end 137.8755 55.1245) (width 0.2) (layer "B.Cu") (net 19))
 (segment (start 108.35 62.023654) (end 110.169154 60.2045) (width 0.2) (layer "B.Cu") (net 19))
 (segment (start 112.04 62.5) (end 110.89 63.65) (width 0.2) (layer "B.Cu") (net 19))
 (segment (start 110.169154 60.2045) (end 130.634484 60.2045) (width 0.2) (layer "B.Cu") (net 19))
 (segment (start 110.89 63.65) (end 109.023654 63.65) (width 0.2) (layer "B.Cu") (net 19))
 (segment (start 130.634484 60.2045) (end 135.714484 55.1245) (width 0.2) (layer "B.Cu") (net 19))
 (segment (start 108.35 62.976346) (end 108.35 62.023654) (width 0.2) (layer "B.Cu") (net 19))
 (segment (start 137.8755 55.1245) (end 148.5 44.5) (width 0.2) (layer "B.Cu") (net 19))
 (segment (start 109.023654 63.65) (end 108.35 62.976346) (width 0.2) (layer "B.Cu") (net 19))
 (segment (start 139.0165 45.9435) (end 142 42.96) (width 0.2) (layer "F.Cu") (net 18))
 (segment (start 136.12 45.9435) (end 139.0165 45.9435) (width 0.2) (layer "F.Cu") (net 18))
 (segment (start 109.8375 59.6225) (end 122.441 59.6225) (width 0.2) (layer "B.Cu") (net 18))
 (segment (start 122.441 59.6225) (end 136.12 45.9435) (width 0.2) (layer "B.Cu") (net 18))
 (segment (start 106.96 62.5) (end 109.8375 59.6225) (width 0.2) (layer "B.Cu") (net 18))
 (segment (start 140.4875 51.178846) (end 140.4875 55.184744) (width 0.2) (layer "F.Cu") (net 25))
 (segment (start 143.15 46.65) (end 143.15 48.516346) (width 0.2) (layer "F.Cu") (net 25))
 (segment (start 128.5825 57.0825) (end 121.5445 50.0445) (width 0.2) (layer "F.Cu") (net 25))
 (segment (start 121.5445 50.0445) (end 112.933 50.0445) (width 0.2) (layer "F.Cu") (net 25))
 (segment (start 142 45.5) (end 143.15 46.65) (width 0.2) (layer "F.Cu") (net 25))
 (segment (start 140.4875 55.184744) (end 138.589744 57.0825) (width 0.2) (layer "F.Cu") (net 25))
 (segment (start 138.589744 57.0825) (end 128.5825 57.0825) (width 0.2) (layer "F.Cu") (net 25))
 (segment (start 112.933 50.0445) (end 106.31 56.6675) (width 0.2) (layer "F.Cu") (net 25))
 (segment (start 143.15 48.516346) (end 140.4875 51.178846) (width 0.2) (layer "F.Cu") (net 25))
 (segment (start 137.1775 52.0025) (end 139.675 54.5) (width 0.2) (layer "F.Cu") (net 8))
 (segment (start 120.88 48.4835) (end 124.399 52.0025) (width 0.2) (layer "F.Cu") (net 8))
 (segment (start 124.399 52.0025) (end 137.1775 52.0025) (width 0.2) (layer "F.Cu") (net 8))
 (segment (start 127.521 57.6645) (end 138.8395 57.6645) (width 0.2) (layer "F.Cu") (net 3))
 (segment (start 120.88 51.0235) (end 127.521 57.6645) (width 0.2) (layer "F.Cu") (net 3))
 (segment (start 138.8395 57.6645) (end 139.675 58.5) (width 0.2) (layer "F.Cu") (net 3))
 (segment (start 120.88 53.5635) (end 130.2165 62.9) (width 0.2) (layer "F.Cu") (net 9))
 (segment (start 130.2165 62.9) (end 139.675 62.9) (width 0.2) (layer "F.Cu") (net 9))
 (segment (start 91.07 56.6675) (end 92.259 57.8565) (width 0.2) (layer "F.Cu") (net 17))
 (segment (start 113.7915 47.5045) (end 132.601 47.5045) (width 0.2) (layer "F.Cu") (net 17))
 (segment (start 104.4245 57.8565) (end 105.121 57.16) (width 0.2) (layer "F.Cu") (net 17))
 (segment (start 105.121 57.16) (end 105.121 56.175) (width 0.2) (layer "F.Cu") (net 17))
 (segment (start 105.121 56.175) (end 113.7915 47.5045) (width 0.2) (layer "F.Cu") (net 17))
 (segment (start 132.601 47.5045) (end 136.12 51.0235) (width 0.2) (layer "F.Cu") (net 17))
 (segment (start 92.259 57.8565) (end 104.4245 57.8565) (width 0.2) (layer "F.Cu") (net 17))
 (segment (start 98.126 58.6435) (end 120.88 58.6435) (width 0.2) (layer "B.Cu") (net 11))
 (segment (start 96.15 56.6675) (end 98.126 58.6435) (width 0.2) (layer "B.Cu") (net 11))
 (segment (start 120.255 55.4785) (end 120.88 56.1035) (width 0.2) (layer "B.Cu") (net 10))
 (segment (start 98.69 56.6675) (end 99.879 55.4785) (width 0.2) (layer "B.Cu") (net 10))
 (segment (start 99.879 55.4785) (end 120.255 55.4785) (width 0.2) (layer "B.Cu") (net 10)))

